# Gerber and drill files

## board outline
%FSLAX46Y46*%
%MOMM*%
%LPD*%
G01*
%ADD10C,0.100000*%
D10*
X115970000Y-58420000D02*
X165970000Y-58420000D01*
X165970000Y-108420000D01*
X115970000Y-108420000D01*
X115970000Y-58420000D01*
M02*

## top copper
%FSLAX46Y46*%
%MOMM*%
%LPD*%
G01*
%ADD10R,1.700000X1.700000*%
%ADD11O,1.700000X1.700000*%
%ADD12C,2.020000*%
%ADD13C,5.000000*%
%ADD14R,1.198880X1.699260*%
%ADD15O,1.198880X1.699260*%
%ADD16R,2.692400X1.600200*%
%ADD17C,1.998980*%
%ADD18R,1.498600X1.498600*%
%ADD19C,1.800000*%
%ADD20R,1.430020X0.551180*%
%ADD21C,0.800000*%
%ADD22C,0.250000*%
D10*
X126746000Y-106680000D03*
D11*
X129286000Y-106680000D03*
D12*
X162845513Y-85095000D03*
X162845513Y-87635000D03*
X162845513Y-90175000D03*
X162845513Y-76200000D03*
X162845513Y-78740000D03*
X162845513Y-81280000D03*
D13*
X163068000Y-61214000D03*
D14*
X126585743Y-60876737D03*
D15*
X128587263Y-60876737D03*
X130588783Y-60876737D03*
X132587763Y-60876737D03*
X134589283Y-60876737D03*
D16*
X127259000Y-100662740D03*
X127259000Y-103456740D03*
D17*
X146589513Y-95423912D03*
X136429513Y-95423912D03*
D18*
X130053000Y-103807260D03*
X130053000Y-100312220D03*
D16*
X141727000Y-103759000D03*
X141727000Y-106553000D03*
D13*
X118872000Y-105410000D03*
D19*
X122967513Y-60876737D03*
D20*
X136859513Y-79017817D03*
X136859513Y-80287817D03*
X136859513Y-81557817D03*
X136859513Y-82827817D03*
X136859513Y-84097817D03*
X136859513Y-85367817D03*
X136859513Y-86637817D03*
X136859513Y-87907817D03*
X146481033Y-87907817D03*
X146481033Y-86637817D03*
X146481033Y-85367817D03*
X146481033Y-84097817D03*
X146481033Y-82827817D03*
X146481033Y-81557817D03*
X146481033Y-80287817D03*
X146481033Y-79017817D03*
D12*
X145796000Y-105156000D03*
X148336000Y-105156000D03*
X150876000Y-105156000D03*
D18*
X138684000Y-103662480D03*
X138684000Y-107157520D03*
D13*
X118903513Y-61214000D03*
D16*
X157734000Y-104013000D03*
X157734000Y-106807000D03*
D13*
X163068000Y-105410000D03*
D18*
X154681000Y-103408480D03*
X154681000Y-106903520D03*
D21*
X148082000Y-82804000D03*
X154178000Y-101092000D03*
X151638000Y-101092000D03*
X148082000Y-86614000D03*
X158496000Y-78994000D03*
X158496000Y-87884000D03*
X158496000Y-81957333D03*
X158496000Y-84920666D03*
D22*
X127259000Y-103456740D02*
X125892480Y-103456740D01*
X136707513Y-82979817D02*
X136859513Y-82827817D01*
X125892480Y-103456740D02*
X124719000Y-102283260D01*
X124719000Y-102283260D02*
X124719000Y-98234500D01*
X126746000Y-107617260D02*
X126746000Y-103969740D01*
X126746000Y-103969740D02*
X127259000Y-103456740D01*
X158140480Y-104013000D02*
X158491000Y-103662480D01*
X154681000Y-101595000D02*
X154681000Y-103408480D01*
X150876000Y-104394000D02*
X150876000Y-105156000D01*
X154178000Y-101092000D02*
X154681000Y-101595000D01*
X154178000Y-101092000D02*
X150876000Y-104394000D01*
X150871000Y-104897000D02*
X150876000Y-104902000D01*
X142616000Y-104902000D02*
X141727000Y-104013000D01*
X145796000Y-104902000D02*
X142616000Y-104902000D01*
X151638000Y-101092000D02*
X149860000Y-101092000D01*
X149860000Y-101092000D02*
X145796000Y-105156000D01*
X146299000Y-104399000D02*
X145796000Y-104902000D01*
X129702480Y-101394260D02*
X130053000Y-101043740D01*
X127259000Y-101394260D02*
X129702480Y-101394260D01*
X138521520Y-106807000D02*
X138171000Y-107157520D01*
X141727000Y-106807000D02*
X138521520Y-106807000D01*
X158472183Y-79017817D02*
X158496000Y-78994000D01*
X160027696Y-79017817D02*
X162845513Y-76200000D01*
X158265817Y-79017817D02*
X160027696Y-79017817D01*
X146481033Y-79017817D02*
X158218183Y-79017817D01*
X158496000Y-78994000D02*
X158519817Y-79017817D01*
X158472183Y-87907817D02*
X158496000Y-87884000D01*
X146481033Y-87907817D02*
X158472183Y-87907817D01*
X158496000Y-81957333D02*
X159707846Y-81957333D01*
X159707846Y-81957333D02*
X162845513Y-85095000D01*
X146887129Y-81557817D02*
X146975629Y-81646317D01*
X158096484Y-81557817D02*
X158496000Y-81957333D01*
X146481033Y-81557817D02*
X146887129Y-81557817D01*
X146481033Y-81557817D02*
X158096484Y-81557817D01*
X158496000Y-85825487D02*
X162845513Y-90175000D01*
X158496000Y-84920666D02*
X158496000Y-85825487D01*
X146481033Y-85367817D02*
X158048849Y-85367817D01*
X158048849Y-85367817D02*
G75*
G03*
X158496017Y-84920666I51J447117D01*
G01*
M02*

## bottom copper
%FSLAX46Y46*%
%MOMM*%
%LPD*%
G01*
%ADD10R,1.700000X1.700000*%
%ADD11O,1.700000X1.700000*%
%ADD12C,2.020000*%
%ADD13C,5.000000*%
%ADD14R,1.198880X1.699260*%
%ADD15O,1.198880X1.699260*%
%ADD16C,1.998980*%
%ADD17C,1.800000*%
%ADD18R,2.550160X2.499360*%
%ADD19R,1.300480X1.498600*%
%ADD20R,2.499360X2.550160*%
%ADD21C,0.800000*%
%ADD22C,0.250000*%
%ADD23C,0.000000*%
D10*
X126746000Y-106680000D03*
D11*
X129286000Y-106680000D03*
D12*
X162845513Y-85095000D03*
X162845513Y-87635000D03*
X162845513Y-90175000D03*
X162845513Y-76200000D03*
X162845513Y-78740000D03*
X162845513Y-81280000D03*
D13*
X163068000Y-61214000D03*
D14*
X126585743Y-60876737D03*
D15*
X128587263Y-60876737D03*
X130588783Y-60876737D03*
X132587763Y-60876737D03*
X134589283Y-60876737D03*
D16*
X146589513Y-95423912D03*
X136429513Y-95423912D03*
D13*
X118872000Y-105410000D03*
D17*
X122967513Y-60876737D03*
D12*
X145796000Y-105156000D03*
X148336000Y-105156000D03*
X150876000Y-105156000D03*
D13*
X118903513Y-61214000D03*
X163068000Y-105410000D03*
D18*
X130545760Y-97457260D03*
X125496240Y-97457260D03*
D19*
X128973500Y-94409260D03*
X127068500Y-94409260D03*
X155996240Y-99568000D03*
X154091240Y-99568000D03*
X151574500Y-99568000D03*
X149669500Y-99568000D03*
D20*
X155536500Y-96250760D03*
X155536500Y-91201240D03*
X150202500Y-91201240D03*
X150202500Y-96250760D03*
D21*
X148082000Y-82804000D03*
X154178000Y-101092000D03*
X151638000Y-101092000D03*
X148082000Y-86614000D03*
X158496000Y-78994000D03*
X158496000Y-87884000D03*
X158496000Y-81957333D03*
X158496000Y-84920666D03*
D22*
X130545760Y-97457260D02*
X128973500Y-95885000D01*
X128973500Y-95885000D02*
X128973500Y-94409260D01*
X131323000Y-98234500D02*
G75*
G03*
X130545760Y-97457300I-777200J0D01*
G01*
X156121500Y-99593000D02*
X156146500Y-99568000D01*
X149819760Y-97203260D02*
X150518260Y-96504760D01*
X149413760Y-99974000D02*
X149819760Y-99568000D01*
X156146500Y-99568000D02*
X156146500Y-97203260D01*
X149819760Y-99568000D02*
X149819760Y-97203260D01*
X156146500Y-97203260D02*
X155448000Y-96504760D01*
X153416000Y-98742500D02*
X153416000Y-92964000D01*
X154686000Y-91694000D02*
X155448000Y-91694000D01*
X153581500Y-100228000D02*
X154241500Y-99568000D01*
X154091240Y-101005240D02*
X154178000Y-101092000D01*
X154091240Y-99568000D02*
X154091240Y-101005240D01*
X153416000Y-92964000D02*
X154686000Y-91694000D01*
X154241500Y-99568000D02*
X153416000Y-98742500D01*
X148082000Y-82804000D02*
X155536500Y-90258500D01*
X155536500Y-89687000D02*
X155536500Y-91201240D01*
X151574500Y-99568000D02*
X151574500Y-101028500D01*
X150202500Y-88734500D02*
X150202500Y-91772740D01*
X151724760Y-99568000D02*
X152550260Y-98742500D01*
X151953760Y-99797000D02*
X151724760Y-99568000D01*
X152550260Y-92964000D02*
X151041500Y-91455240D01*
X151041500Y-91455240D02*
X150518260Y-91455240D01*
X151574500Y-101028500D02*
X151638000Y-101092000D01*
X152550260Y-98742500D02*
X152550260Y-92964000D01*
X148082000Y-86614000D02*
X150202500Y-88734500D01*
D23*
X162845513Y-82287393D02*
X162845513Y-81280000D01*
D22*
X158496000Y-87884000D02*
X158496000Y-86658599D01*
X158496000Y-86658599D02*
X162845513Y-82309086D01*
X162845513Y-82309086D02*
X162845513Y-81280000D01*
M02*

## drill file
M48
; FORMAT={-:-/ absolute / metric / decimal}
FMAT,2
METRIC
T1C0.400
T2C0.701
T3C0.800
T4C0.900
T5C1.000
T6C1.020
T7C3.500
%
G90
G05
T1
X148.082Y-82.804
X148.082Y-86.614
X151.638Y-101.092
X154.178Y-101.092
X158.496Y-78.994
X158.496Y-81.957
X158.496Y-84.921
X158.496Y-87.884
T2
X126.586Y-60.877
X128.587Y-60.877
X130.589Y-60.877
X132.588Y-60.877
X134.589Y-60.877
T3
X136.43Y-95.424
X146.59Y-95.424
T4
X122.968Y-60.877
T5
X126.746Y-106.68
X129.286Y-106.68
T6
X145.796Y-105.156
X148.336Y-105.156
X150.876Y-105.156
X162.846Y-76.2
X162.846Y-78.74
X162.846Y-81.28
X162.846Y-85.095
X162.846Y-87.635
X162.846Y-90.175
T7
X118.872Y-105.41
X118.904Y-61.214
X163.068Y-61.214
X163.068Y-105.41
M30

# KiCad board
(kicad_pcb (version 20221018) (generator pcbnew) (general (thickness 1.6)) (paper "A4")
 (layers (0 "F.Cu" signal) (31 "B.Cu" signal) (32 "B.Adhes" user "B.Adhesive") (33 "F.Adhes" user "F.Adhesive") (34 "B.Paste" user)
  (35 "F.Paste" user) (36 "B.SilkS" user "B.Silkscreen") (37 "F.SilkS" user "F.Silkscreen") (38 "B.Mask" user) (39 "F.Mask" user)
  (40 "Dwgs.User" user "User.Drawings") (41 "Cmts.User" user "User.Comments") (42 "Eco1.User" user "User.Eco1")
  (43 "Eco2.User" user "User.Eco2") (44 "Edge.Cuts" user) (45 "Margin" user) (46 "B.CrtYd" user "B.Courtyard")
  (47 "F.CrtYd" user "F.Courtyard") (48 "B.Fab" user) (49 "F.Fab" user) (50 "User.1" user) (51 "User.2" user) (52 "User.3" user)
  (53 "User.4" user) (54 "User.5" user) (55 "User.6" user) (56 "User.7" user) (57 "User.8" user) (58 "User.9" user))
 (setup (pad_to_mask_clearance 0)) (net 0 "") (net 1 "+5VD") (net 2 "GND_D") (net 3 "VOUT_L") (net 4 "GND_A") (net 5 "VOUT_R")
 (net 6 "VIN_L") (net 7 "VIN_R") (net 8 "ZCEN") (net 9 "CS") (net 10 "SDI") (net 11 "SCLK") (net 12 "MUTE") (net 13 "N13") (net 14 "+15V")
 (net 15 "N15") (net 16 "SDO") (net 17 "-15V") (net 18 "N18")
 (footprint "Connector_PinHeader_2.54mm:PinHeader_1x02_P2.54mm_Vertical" (layer "F.Cu") (at 126.746 106.68 90)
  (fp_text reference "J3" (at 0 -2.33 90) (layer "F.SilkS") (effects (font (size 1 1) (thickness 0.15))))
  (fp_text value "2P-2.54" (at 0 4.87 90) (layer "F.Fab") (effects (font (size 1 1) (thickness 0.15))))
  (pad "1" thru_hole rect (at 0 0 90) (size 1.7 1.7) (drill 1) (layers "*.Cu" "*.Mask") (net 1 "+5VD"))
  (pad "2" thru_hole oval (at 0 2.54 90) (size 1.7 1.7) (drill 1) (layers "*.Cu" "*.Mask") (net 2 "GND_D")))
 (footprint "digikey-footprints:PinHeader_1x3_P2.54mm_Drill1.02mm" (layer "F.Cu") (at 162.845513 85.095 -90)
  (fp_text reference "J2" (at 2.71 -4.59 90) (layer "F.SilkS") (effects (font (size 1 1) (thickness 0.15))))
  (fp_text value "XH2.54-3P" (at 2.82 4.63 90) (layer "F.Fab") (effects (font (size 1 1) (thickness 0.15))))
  (pad "1" thru_hole circle (at 0 0 270) (size 2.02 2.02) (drill 1.02) (layers "*.Cu" "*.Mask") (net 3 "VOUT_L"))
  (pad "2" thru_hole circle (at 2.54 0 270) (size 2.02 2.02) (drill 1.02) (layers "*.Cu" "*.Mask") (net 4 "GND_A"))
  (pad "3" thru_hole circle (at 5.08 0 270) (size 2.02 2.02) (drill 1.02) (layers "*.Cu" "*.Mask") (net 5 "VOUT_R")))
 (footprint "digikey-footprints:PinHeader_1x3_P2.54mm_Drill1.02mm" (layer "F.Cu") (at 162.845513 76.2 -90)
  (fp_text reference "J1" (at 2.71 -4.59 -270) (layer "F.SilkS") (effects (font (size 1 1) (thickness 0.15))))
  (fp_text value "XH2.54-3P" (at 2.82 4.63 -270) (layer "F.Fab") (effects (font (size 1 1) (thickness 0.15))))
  (pad "1" thru_hole circle (at 0 0 270) (size 2.02 2.02) (drill 1.02) (layers "*.Cu" "*.Mask") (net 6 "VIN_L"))
  (pad "2" thru_hole circle (at 2.54 0 270) (size 2.02 2.02) (drill 1.02) (layers "*.Cu" "*.Mask") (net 4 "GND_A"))
  (pad "3" thru_hole circle (at 5.08 0 270) (size 2.02 2.02) (drill 1.02) (layers "*.Cu" "*.Mask") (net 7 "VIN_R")))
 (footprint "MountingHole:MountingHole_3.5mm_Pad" (layer "F.Cu") (at 163.068 61.214)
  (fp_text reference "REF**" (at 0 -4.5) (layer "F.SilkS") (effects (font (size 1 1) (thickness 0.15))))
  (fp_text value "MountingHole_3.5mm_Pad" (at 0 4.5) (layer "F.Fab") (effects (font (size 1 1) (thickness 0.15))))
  (pad "1" thru_hole circle (at 0 0) (size 5 5) (drill 3.5) (layers "*.Cu" "*.Mask" "F.SilkS")))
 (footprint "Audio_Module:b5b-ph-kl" (layer "F.Cu") (at 130.588783 60.876737)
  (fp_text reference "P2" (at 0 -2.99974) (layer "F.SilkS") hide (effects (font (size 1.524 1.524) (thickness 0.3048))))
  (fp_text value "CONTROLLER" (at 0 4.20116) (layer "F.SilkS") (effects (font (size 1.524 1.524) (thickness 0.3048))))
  (pad "1" thru_hole rect (at -4.00304 0) (size 1.19888 1.69926) (drill 0.70104) (layers "*.Cu" "*.Mask" "F.SilkS") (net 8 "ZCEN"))
  (pad "2" thru_hole oval (at -2.00152 0) (size 1.19888 1.69926) (drill 0.70104) (layers "*.Cu" "*.Mask" "F.SilkS") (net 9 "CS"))
  (pad "3" thru_hole oval (at 0 0) (size 1.19888 1.69926) (drill 0.70104) (layers "*.Cu" "*.Mask" "F.SilkS") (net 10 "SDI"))
  (pad "4" thru_hole oval (at 1.99898 0) (size 1.19888 1.69926) (drill 0.70104) (layers "*.Cu" "*.Mask" "F.SilkS") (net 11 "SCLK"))
  (pad "5" thru_hole oval (at 4.0005 0) (size 1.19888 1.69926) (drill 0.70104) (layers "*.Cu" "*.Mask" "F.SilkS") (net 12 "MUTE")))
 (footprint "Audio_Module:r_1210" (layer "F.Cu") (at 127.259 102.05974 90)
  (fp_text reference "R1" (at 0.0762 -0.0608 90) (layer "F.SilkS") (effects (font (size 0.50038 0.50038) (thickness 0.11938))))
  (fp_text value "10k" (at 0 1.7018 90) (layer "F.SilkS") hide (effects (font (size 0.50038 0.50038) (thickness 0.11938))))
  (pad "1" smd rect (at 1.397 0 90) (size 1.6002 2.6924) (layers "F.Cu" "F.Paste" "F.Mask") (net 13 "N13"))
  (pad "2" smd rect (at -1.397 0 90) (size 1.6002 2.6924) (layers "F.Cu" "F.Paste" "F.Mask") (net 1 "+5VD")))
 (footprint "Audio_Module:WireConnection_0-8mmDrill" (layer "F.Cu") (at 146.589513 95.423912 180)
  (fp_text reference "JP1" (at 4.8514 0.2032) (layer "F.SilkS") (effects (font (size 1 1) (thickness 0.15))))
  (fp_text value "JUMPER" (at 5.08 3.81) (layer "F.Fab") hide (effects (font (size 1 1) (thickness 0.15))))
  (pad "1" thru_hole circle (at 0 0 180) (size 1.99898 1.99898) (drill 0.8001) (layers "*.Cu" "*.Mask" "F.SilkS") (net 4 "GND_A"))
  (pad "2" thru_hole circle (at 10.16 0 180) (size 1.99898 1.99898) (drill 0.8001) (layers "*.Cu" "*.Mask" "F.SilkS") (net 2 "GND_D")))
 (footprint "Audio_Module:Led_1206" (layer "F.Cu") (at 130.053 102.05974 90)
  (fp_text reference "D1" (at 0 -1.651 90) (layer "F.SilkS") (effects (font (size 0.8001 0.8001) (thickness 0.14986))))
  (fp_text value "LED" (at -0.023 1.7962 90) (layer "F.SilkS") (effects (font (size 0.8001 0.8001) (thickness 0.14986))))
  (pad "1" smd rect (at -1.74752 0 90) (size 1.4986 1.4986) (layers "F.Cu" "F.Paste" "F.Mask") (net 2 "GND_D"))
  (pad "2" smd rect (at 1.74752 0 90) (size 1.4986 1.4986) (layers "F.Cu" "F.Paste" "F.Mask") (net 13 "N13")))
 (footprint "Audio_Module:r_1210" (layer "F.Cu") (at 141.727 105.156 90)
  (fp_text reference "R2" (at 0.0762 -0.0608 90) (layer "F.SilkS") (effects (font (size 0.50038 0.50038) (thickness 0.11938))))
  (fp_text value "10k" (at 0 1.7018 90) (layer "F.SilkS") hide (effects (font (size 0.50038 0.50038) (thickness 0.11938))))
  (pad "1" smd rect (at 1.397 0 90) (size 1.6002 2.6924) (layers "F.Cu" "F.Paste" "F.Mask") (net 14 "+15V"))
  (pad "2" smd rect (at -1.397 0 90) (size 1.6002 2.6924) (layers "F.Cu" "F.Paste" "F.Mask") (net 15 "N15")))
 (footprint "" (layer "F.Cu") (at 118.618 105.41)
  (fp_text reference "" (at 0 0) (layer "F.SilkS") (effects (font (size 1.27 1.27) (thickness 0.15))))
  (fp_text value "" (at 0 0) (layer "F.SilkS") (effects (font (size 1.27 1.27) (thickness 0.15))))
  (pad "1" thru_hole circle (at 0.254 0) (size 5 5) (drill 3.5) (layers "*.Cu" "*.Mask" "F.SilkS")))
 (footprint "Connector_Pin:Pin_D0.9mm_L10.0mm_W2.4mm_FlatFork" (layer "F.Cu") (at 122.967513 60.876737)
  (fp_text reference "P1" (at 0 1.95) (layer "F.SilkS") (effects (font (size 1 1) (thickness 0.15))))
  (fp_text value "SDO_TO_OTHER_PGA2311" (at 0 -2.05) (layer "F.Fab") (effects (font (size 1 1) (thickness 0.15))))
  (pad "1" thru_hole circle (at 0 0) (size 1.8 1.8) (drill 0.9) (layers "*.Cu" "*.Mask") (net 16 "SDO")))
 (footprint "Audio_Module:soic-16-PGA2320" (layer "F.Cu") (at 141.670273 83.462817)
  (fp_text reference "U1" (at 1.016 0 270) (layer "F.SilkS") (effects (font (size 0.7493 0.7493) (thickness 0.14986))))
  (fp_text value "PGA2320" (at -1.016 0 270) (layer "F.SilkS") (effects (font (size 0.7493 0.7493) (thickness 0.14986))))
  (pad "1" smd rect (at -4.81076 -4.445 270) (size 0.55118 1.43002) (layers "F.Cu" "F.Paste" "F.Mask") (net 8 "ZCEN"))
  (pad "2" smd rect (at -4.81076 -3.175 270) (size 0.55118 1.43002) (layers "F.Cu" "F.Paste" "F.Mask") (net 9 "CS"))
  (pad "3" smd rect (at -4.81076 -1.905 270) (size 0.55118 1.43002) (layers "F.Cu" "F.Paste" "F.Mask") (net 10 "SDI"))
  (pad "4" smd rect (at -4.81076 -0.635 270) (size 0.55118 1.43002) (layers "F.Cu" "F.Paste" "F.Mask") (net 1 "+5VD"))
  (pad "5" smd rect (at -4.81076 0.635 270) (size 0.55118 1.43002) (layers "F.Cu" "F.Paste" "F.Mask") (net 2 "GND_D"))
  (pad "6" smd rect (at -4.81076 1.905 270) (size 0.55118 1.43002) (layers "F.Cu" "F.Paste" "F.Mask") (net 11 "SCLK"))
  (pad "7" smd rect (at -4.81076 3.175 270) (size 0.55118 1.43002) (layers "F.Cu" "F.Paste" "F.Mask") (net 16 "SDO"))
  (pad "8" smd rect (at -4.81076 4.445 270) (size 0.55118 1.43002) (layers "F.Cu" "F.Paste" "F.Mask") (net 12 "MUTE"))
  (pad "9" smd rect (at 4.81076 4.445 270) (size 0.55118 1.43002) (layers "F.Cu" "F.Paste" "F.Mask") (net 7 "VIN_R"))
  (pad "10" smd rect (at 4.81076 3.175 270) (size 0.55118 1.43002) (layers "F.Cu" "F.Paste" "F.Mask") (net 4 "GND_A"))
  (pad "11" smd rect (at 4.81076 1.905 270) (size 0.55118 1.43002) (layers "F.Cu" "F.Paste" "F.Mask") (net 5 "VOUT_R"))
  (pad "12" smd rect (at 4.81076 0.635 270) (size 0.55118 1.43002) (layers "F.Cu" "F.Paste" "F.Mask") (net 14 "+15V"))
  (pad "13" smd rect (at 4.81076 -0.635 270) (size 0.55118 1.43002) (layers "F.Cu" "F.Paste" "F.Mask") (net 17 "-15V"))
  (pad "14" smd rect (at 4.81076 -1.905 270) (size 0.55118 1.43002) (layers "F.Cu" "F.Paste" "F.Mask") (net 3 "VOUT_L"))
  (pad "15" smd rect (at 4.81076 -3.175 270) (size 0.55118 1.43002) (layers "F.Cu" "F.Paste" "F.Mask") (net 4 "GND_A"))
  (pad "16" smd rect (at 4.81076 -4.445 270) (size 0.55118 1.43002) (layers "F.Cu" "F.Paste" "F.Mask") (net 6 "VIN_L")))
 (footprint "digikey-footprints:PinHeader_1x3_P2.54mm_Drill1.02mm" (layer "F.Cu") (at 145.796 105.156)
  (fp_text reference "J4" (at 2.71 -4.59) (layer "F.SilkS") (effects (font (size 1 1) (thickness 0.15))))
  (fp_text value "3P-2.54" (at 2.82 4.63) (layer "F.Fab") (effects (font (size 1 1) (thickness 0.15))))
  (pad "1" thru_hole circle (at 0 0) (size 2.02 2.02) (drill 1.02) (layers "*.Cu" "*.Mask") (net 14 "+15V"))
  (pad "2" thru_hole circle (at 2.54 0) (size 2.02 2.02) (drill 1.02) (layers "*.Cu" "*.Mask") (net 4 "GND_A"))
  (pad "3" thru_hole circle (at 5.08 0) (size 2.02 2.02) (drill 1.02) (layers "*.Cu" "*.Mask") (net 17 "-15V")))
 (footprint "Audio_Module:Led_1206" (layer "F.Cu") (at 138.684 105.41 -90)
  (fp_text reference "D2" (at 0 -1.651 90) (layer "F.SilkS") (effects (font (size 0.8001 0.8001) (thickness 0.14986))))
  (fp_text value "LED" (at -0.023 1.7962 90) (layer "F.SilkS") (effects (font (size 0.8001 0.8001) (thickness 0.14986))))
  (pad "1" smd rect (at -1.74752 0 270) (size 1.4986 1.4986) (layers "F.Cu" "F.Paste" "F.Mask") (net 4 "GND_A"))
  (pad "2" smd rect (at 1.74752 0 270) (size 1.4986 1.4986) (layers "F.Cu" "F.Paste" "F.Mask") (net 15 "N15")))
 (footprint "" (layer "F.Cu") (at 118.903513 61.214)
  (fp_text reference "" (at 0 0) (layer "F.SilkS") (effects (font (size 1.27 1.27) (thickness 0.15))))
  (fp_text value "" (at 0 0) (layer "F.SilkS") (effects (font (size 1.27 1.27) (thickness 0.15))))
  (pad "1" thru_hole circle (at 0 0) (size 5 5) (drill 3.5) (layers "*.Cu" "*.Mask" "F.SilkS")))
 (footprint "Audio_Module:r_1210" (layer "F.Cu") (at 157.734 105.41 90)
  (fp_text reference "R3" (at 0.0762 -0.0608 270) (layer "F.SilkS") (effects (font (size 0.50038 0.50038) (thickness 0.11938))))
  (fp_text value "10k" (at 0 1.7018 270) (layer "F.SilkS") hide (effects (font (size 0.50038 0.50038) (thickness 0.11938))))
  (pad "1" smd rect (at 1.397 0 90) (size 1.6002 2.6924) (layers "F.Cu" "F.Paste" "F.Mask") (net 4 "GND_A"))
  (pad "2" smd rect (at -1.397 0 90) (size 1.6002 2.6924) (layers "F.Cu" "F.Paste" "F.Mask") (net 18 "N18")))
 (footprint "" (layer "F.Cu") (at 163.068 105.918)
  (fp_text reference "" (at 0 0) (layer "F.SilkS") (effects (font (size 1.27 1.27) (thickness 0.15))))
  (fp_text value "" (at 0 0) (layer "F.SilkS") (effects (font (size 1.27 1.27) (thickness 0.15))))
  (pad "1" thru_hole circle (at 0 -0.508) (size 5 5) (drill 3.5) (layers "*.Cu" "*.Mask" "F.SilkS")))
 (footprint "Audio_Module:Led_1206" (layer "F.Cu") (at 154.681 105.156 -90)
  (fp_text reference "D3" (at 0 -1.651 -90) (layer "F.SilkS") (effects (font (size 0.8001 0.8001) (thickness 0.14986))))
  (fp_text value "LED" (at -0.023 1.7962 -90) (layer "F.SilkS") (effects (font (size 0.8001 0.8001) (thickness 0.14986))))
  (pad "1" smd rect (at -1.74752 0 270) (size 1.4986 1.4986) (layers "F.Cu" "F.Paste" "F.Mask") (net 17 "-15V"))
  (pad "2" smd rect (at 1.74752 0 270) (size 1.4986 1.4986) (layers "F.Cu" "F.Paste" "F.Mask") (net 18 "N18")))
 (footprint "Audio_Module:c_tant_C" (layer "B.Cu") (at 128.021 97.45726)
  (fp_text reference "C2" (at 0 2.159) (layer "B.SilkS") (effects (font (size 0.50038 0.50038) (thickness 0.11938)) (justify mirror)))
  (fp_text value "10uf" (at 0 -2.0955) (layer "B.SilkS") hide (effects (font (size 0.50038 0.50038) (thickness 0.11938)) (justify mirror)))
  (pad "1" smd rect (at 2.52476 0) (size 2.55016 2.49936) (layers "B.Cu" "B.Paste" "B.Mask") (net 1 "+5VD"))
  (pad "2" smd rect (at -2.52476 0) (size 2.55016 2.49936) (layers "B.Cu" "B.Paste" "B.Mask") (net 2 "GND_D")))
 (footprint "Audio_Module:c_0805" (layer "B.Cu") (at 128.021 94.40926)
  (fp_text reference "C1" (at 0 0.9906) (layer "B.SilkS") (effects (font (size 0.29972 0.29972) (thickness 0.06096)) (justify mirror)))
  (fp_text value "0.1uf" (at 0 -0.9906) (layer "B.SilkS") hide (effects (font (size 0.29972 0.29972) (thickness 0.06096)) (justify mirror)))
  (pad "1" smd rect (at 0.9525 0) (size 1.30048 1.4986) (layers "B.Cu" "B.Paste" "B.Mask") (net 1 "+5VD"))
  (pad "2" smd rect (at -0.9525 0) (size 1.30048 1.4986) (layers "B.Cu" "B.Paste" "B.Mask") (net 2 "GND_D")))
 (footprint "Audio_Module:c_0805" (layer "B.Cu") (at 155.04374 99.568)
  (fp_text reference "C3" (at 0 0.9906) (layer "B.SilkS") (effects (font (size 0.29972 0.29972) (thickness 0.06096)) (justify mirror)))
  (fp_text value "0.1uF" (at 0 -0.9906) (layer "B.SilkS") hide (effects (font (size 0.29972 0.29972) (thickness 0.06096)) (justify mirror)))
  (pad "1" smd rect (at 0.9525 0) (size 1.30048 1.4986) (layers "B.Cu" "B.Paste" "B.Mask") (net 4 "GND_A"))
  (pad "2" smd rect (at -0.9525 0) (size 1.30048 1.4986) (layers "B.Cu" "B.Paste" "B.Mask") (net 17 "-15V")))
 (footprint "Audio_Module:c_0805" (layer "B.Cu") (at 150.622 99.568)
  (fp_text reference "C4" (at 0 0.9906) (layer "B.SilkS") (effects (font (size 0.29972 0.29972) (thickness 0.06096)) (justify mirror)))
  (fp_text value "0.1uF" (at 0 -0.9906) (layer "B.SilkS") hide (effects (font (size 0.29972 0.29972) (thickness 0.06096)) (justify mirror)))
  (pad "1" smd rect (at 0.9525 0) (size 1.30048 1.4986) (layers "B.Cu" "B.Paste" "B.Mask") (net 14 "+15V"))
  (pad "2" smd rect (at -0.9525 0) (size 1.30048 1.4986) (layers "B.Cu" "B.Paste" "B.Mask") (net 4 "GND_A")))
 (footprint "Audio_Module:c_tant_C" (layer "B.Cu") (at 155.5365 93.726 -90)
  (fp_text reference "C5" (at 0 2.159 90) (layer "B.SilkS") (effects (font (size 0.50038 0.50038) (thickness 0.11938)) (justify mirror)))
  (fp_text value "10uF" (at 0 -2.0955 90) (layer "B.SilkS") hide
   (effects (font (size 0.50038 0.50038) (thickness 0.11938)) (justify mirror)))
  (pad "1" smd rect (at 2.52476 0 270) (size 2.55016 2.49936) (layers "B.Cu" "B.Paste" "B.Mask") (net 4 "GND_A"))
  (pad "2" smd rect (at -2.52476 0 270) (size 2.55016 2.49936) (layers "B.Cu" "B.Paste" "B.Mask") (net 17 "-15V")))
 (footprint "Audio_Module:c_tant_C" (layer "B.Cu") (at 150.2025 93.726 90)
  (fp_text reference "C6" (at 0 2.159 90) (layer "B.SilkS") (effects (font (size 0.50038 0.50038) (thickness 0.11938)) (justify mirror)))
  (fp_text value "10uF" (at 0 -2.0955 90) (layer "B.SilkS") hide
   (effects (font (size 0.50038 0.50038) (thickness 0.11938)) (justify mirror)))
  (pad "1" smd rect (at 2.52476 0 90) (size 2.55016 2.49936) (layers "B.Cu" "B.Paste" "B.Mask") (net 14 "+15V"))
  (pad "2" smd rect (at -2.52476 0 90) (size 2.55016 2.49936) (layers "B.Cu" "B.Paste" "B.Mask") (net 4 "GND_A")))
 (gr_rect (start 115.97 58.42) (end 165.97 108.42) (stroke (width 0.1) (type default)) (fill none) (layer "Edge.Cuts"))
 (gr_rect (start 162.56 97.79) (end 162.56 97.79) (stroke (width 0.1) (type default)) (fill none) (layer "Edge.Cuts"))
 (segment (start 127.259 103.45674) (end 125.89248 103.45674) (width 0.25) (layer "F.Cu") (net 1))
 (segment (start 136.707513 82.979817) (end 136.859513 82.827817) (width 0.25) (layer "F.Cu") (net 1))
 (segment (start 125.89248 103.45674) (end 124.719 102.28326) (width 0.25) (layer "F.Cu") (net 1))
 (segment (start 124.719 102.28326) (end 124.719 98.2345) (width 0.25) (layer "F.Cu") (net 1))
 (segment (start 126.746 107.61726) (end 126.746 103.96974) (width 0.25) (layer "F.Cu") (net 1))
 (segment (start 126.746 103.96974) (end 127.259 103.45674) (width 0.25) (layer "F.Cu") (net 1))
 (segment (start 130.54576 97.45726) (end 128.9735 95.885) (width 0.25) (layer "B.Cu") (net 1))
 (segment (start 128.9735 95.885) (end 128.9735 94.40926) (width 0.25) (layer "B.Cu") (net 1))
 (arc (start 131.323 98.2345) (mid 131.095352 97.684908) (end 130.54576 97.45726) (width 0.25) (layer "B.Cu") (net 1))
 (segment (start 158.14048 104.013) (end 158.491 103.66248) (width 0.25) (layer "F.Cu") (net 4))
 (segment (start 156.1215 99.593) (end 156.1465 99.568) (width 0.25) (layer "B.Cu") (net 4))
 (segment (start 149.81976 97.20326) (end 150.51826 96.50476) (width 0.25) (layer "B.Cu") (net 4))
 (segment (start 149.41376 99.974) (end 149.81976 99.568) (width 0.25) (layer "B.Cu") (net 4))
 (segment (start 156.1465 99.568) (end 156.1465 97.20326) (width 0.25) (layer "B.Cu") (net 4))
 (segment (start 149.81976 99.568) (end 149.81976 97.20326) (width 0.25) (layer "B.Cu") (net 4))
 (segment (start 156.1465 97.20326) (end 155.448 96.50476) (width 0.25) (layer "B.Cu") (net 4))
 (segment (start 154.681 101.595) (end 154.681 103.40848) (width 0.25) (layer "F.Cu") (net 17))
 (segment (start 150.876 104.394) (end 150.876 105.156) (width 0.25) (layer "F.Cu") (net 17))
 (segment (start 154.178 101.092) (end 154.681 101.595) (width 0.25) (layer "F.Cu") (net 17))
 (segment (start 154.178 101.092) (end 150.876 104.394) (width 0.25) (layer "F.Cu") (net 17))
 (segment (start 150.871 104.897) (end 150.876 104.902) (width 0.25) (layer "F.Cu") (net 17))
 (via (at 148.082 82.804) (size 0.8) (drill 0.4) (layers "F.Cu" "B.Cu") (free) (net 17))
 (via (at 154.178 101.092) (size 0.8) (drill 0.4) (layers "F.Cu" "B.Cu") (free) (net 17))
 (segment (start 153.416 98.7425) (end 153.416 92.964) (width 0.25) (layer "B.Cu") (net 17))
 (segment (start 154.686 91.694) (end 155.448 91.694) (width 0.25) (layer "B.Cu") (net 17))
 (segment (start 153.5815 100.228) (end 154.2415 99.568) (width 0.25) (layer "B.Cu") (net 17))
 (segment (start 154.09124 101.00524) (end 154.178 101.092) (width 0.25) (layer "B.Cu") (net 17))
 (segment (start 154.09124 99.568) (end 154.09124 101.00524) (width 0.25) (layer "B.Cu") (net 17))
 (segment (start 153.416 92.964) (end 154.686 91.694) (width 0.25) (layer "B.Cu") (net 17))
 (segment (start 154.2415 99.568) (end 153.416 98.7425) (width 0.25) (layer "B.Cu") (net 17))
 (segment (start 148.082 82.804) (end 155.5365 90.2585) (width 0.25) (layer "B.Cu") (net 17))
 (segment (start 155.5365 89.687) (end 155.5365 91.20124) (width 0.25) (layer "B.Cu") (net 17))
 (segment (start 142.616 104.902) (end 141.727 104.013) (width 0.25) (layer "F.Cu") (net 14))
 (segment (start 145.796 104.902) (end 142.616 104.902) (width 0.25) (layer "F.Cu") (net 14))
 (segment (start 151.638 101.092) (end 149.86 101.092) (width 0.25) (layer "F.Cu") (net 14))
 (segment (start 149.86 101.092) (end 145.796 105.156) (width 0.25) (layer "F.Cu") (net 14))
 (segment (start 146.299 104.399) (end 145.796 104.902) (width 0.25) (layer "F.Cu") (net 14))
 (via (at 151.638 101.092) (size 0.8) (drill 0.4) (layers "F.Cu" "B.Cu") (free) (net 14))
 (via (at 148.082 86.614) (size 0.8) (drill 0.4) (layers "F.Cu" "B.Cu") (free) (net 14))
 (segment (start 151.5745 99.568) (end 151.5745 101.0285) (width 0.25) (layer "B.Cu") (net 14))
 (segment (start 150.2025 88.7345) (end 150.2025 91.77274) (width 0.25) (layer "B.Cu") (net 14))
 (segment (start 151.72476 99.568) (end 152.55026 98.7425) (width 0.25) (layer "B.Cu") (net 14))
 (segment (start 151.95376 99.797) (end 151.72476 99.568) (width 0.25) (layer "B.Cu") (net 14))
 (segment (start 152.55026 92.964) (end 151.0415 91.45524) (width 0.25) (layer "B.Cu") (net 14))
 (segment (start 151.0415 91.45524) (end 150.51826 91.45524) (width 0.25) (layer "B.Cu") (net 14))
 (segment (start 151.5745 101.0285) (end 151.638 101.092) (width 0.25) (layer "B.Cu") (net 14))
 (segment (start 152.55026 98.7425) (end 152.55026 92.964) (width 0.25) (layer "B.Cu") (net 14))
 (segment (start 148.082 86.614) (end 150.2025 88.7345) (width 0.25) (layer "B.Cu") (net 14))
 (segment (start 129.70248 101.39426) (end 130.053 101.04374) (width 0.25) (layer "F.Cu") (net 13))
 (segment (start 127.259 101.39426) (end 129.70248 101.39426) (width 0.25) (layer "F.Cu") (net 13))
 (segment (start 138.52152 106.807) (end 138.171 107.15752) (width 0.25) (layer "F.Cu") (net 15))
 (segment (start 141.727 106.807) (end 138.52152 106.807) (width 0.25) (layer "F.Cu") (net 15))
 (segment (start 158.472183 79.017817) (end 158.496 78.994) (width 0.25) (layer "F.Cu") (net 6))
 (segment (start 160.027696 79.017817) (end 162.845513 76.2) (width 0.25) (layer "F.Cu") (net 6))
 (segment (start 158.265817 79.017817) (end 160.027696 79.017817) (width 0.25) (layer "F.Cu") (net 6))
 (segment (start 146.481033 79.017817) (end 158.218183 79.017817) (width 0.25) (layer "F.Cu") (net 6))
 (segment (start 158.496 78.994) (end 158.519817 79.017817) (width 0.25) (layer "F.Cu") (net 6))
 (via (at 158.496 78.994) (size 0.8) (drill 0.4) (layers "F.Cu" "B.Cu") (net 6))
 (segment (start 158.472183 87.907817) (end 158.496 87.884) (width 0.25) (layer "F.Cu") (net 7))
 (segment (start 146.481033 87.907817) (end 158.472183 87.907817) (width 0.25) (layer "F.Cu") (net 7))
 (via (at 158.496 87.884) (size 0.8) (drill 0.4) (layers "F.Cu" "B.Cu") (free) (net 7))
 (segment (start 162.845513 82.287393) (end 162.845513 81.28) (width 0) (layer "B.Cu") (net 7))
 (segment (start 158.496 87.884) (end 158.496 86.658599) (width 0.25) (layer "B.Cu") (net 7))
 (segment (start 158.496 86.658599) (end 162.845513 82.309086) (width 0.25) (layer "B.Cu") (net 7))
 (segment (start 162.845513 82.309086) (end 162.845513 81.28) (width 0.25) (layer "B.Cu") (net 7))
 (segment (start 158.496 81.957333) (end 159.707846 81.957333) (width 0.25) (layer "F.Cu") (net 3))
 (segment (start 159.707846 81.957333) (end 162.845513 85.095) (width 0.25) (layer "F.Cu") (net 3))
 (segment (start 146.887129 81.557817) (end 146.975629 81.646317) (width 0.25) (layer "F.Cu") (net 3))
 (segment (start 158.096484 81.557817) (end 158.496 81.957333) (width 0.25) (layer "F.Cu") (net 3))
 (segment (start 146.481033 81.557817) (end 146.887129 81.557817) (width 0.25) (layer "F.Cu") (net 3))
 (segment (start 146.481033 81.557817) (end 158.096484 81.557817) (width 0.25) (layer "F.Cu") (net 3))
 (via (at 158.496 81.957333) (size 0.8) (drill 0.4) (layers "F.Cu" "B.Cu") (free) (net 3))
 (segment (start 158.496 85.825487) (end 162.845513 90.175) (width 0.25) (layer "F.Cu") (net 5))
 (segment (start 158.496 84.920666) (end 158.496 85.825487) (width 0.25) (layer "F.Cu") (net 5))
 (segment (start 146.481033 85.367817) (end 158.048849 85.367817) (width 0.25) (layer "F.Cu") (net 5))
 (via (at 158.496 84.920666) (size 0.8) (drill 0.4) (layers "F.Cu" "B.Cu") (free) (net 5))
 (arc (start 158.048849 85.367817) (mid 158.365033 85.23685) (end 158.496 84.920666) (width 0.25) (layer "F.Cu") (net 5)))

